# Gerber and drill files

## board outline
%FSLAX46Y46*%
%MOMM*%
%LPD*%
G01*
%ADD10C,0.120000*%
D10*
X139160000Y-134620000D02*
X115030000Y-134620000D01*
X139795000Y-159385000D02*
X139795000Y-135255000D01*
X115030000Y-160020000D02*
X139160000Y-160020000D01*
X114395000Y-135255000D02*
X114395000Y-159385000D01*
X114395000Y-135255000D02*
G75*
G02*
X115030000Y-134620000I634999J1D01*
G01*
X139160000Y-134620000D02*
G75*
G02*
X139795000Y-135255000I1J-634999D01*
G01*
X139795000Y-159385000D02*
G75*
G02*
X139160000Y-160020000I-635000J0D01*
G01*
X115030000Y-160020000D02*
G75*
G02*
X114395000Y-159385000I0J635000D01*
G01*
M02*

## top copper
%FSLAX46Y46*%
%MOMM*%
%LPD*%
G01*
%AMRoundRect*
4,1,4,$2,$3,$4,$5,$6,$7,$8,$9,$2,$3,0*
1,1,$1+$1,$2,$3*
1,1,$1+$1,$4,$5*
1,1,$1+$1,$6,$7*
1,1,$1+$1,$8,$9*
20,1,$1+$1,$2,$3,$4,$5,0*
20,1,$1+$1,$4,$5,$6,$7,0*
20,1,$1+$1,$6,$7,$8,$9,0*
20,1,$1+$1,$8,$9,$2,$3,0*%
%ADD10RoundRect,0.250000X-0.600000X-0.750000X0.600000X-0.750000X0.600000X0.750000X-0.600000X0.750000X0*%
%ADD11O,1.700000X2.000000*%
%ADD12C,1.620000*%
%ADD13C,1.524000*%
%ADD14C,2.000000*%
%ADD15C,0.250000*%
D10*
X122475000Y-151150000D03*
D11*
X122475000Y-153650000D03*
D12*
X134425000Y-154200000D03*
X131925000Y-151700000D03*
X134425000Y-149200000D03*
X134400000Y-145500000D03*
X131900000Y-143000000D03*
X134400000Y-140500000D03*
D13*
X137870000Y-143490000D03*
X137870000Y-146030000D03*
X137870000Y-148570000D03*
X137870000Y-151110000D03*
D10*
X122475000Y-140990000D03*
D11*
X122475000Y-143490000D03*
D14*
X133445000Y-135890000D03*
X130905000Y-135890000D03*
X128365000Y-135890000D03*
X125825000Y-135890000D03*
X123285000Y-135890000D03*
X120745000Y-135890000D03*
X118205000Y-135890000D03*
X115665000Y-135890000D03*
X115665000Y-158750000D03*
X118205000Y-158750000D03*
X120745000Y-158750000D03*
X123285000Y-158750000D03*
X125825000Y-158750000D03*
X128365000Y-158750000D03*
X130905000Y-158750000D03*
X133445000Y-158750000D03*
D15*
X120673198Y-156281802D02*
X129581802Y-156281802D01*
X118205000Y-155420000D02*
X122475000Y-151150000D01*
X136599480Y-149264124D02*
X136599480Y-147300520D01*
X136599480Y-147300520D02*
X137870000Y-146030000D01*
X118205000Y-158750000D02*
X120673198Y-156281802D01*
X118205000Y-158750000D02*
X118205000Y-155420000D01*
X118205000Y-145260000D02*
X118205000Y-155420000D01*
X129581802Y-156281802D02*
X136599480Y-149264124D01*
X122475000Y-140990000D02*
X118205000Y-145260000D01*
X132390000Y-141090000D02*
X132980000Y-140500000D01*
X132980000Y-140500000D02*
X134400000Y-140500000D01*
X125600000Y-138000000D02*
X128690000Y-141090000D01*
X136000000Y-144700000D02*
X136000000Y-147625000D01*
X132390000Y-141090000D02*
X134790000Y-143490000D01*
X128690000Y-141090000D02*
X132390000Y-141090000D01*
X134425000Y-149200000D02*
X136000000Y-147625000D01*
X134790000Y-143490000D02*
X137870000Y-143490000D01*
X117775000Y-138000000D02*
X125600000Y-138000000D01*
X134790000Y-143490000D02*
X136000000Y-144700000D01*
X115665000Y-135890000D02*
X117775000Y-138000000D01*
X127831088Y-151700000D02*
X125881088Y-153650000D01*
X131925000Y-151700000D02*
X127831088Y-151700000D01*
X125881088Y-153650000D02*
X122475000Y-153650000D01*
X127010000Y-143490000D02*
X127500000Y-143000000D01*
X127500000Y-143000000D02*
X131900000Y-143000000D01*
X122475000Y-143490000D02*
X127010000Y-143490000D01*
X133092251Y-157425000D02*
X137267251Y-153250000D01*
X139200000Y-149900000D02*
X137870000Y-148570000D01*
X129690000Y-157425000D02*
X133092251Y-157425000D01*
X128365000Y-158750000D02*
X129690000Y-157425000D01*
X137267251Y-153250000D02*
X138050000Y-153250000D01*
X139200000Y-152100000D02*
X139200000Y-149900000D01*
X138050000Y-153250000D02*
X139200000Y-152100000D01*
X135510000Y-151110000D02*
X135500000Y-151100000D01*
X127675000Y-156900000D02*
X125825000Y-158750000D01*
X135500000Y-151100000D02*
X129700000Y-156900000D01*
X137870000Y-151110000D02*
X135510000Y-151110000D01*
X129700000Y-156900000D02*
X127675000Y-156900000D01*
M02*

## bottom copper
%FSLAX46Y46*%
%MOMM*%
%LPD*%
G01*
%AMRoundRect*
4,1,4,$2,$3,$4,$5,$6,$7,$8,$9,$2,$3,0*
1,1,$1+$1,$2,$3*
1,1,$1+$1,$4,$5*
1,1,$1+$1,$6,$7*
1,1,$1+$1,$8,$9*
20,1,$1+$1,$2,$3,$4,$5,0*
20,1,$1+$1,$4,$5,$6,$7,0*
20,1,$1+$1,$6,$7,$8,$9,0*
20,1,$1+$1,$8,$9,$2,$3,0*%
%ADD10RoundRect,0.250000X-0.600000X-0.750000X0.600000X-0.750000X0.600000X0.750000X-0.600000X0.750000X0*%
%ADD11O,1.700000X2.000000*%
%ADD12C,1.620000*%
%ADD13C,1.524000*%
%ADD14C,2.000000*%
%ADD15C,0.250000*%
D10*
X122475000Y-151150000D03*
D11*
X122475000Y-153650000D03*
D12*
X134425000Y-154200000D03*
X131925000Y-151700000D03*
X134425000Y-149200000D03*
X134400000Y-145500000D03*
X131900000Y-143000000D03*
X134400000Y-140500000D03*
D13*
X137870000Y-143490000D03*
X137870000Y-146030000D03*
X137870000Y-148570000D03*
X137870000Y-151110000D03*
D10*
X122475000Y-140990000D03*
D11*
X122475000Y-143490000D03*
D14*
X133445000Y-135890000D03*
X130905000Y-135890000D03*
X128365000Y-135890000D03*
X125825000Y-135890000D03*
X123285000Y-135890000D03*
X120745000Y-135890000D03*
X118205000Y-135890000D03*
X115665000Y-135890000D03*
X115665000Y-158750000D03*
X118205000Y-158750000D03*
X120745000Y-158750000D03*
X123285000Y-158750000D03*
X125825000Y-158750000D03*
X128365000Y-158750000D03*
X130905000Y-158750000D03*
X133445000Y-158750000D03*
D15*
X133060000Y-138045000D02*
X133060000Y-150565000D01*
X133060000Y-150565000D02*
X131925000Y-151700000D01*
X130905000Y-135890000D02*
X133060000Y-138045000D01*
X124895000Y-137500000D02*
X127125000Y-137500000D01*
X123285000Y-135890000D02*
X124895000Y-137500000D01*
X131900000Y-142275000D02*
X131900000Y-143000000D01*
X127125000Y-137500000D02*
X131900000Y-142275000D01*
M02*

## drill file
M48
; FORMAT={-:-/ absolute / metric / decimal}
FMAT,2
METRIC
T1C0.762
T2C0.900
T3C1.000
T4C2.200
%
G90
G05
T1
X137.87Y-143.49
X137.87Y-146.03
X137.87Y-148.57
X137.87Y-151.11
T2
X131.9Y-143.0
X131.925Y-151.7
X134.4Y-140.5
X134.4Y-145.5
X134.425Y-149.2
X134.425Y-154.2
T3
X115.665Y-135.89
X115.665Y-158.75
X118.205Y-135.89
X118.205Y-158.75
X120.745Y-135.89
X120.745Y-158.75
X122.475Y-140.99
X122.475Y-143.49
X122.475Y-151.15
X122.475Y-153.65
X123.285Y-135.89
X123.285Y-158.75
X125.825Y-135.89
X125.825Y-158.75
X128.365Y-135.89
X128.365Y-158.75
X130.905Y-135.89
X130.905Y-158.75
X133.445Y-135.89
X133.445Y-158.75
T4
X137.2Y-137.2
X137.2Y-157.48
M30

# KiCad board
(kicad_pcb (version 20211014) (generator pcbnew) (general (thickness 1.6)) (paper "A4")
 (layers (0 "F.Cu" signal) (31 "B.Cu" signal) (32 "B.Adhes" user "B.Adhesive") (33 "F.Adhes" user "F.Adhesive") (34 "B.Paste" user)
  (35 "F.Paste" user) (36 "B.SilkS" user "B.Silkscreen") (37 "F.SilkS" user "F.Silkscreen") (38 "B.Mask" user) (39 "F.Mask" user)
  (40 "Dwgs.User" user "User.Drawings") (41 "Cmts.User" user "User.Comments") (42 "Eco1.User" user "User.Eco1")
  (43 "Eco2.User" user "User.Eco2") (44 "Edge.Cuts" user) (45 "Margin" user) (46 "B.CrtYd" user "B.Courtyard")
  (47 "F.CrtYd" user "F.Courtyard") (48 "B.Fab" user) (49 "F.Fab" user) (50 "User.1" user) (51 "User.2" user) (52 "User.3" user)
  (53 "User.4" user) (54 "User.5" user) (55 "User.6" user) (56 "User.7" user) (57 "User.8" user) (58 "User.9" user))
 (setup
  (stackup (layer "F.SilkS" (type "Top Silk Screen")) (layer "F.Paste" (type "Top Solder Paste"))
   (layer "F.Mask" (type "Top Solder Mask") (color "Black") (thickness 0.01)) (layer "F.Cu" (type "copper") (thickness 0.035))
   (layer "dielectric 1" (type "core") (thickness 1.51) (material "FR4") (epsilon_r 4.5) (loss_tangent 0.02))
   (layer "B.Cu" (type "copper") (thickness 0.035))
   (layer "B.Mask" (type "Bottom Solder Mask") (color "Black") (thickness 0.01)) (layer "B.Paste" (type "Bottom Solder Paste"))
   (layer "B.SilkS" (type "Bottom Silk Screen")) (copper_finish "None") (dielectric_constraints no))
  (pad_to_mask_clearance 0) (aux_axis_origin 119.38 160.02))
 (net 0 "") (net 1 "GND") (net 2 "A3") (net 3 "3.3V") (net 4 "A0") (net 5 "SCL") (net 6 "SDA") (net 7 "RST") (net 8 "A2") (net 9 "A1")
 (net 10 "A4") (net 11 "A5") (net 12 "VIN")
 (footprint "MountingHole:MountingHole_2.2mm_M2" (layer "F.Cu") (at 137.2 137.2)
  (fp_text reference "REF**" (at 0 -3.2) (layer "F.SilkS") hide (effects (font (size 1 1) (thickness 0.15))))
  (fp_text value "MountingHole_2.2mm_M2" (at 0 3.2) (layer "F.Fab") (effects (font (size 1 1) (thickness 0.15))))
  (pad "" np_thru_hole circle (at 0 0) (size 2.2 2.2) (drill 2.2) (layers *.Cu *.Mask)))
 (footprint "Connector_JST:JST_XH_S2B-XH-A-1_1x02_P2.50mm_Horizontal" (layer "F.Cu") (at 114.375 152.4 -90)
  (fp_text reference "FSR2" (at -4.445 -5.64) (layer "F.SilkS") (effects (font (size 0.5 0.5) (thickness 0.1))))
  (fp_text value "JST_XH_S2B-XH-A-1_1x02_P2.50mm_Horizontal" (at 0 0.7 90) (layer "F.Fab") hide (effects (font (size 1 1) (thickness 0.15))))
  (pad "1" thru_hole roundrect (at -1.25 -8.1) (size 1.7 2) (drill 1) (layers *.Cu *.Mask) (roundrect_rratio 0.1470588235) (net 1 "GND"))
  (pad "2" thru_hole oval (at 1.25 -8.1) (size 1.7 2) (drill 1) (layers *.Cu *.Mask) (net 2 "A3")))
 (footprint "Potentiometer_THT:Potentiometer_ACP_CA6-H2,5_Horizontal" (layer "F.Cu") (at 134.425 154.2 180)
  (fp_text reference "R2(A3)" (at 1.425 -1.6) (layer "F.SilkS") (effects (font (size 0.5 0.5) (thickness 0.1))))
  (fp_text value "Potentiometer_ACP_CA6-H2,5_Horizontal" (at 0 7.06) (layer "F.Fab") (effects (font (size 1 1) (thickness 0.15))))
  (pad "1" thru_hole circle (at 0 0 180) (size 1.62 1.62) (drill 0.9) (layers *.Cu *.Mask))
  (pad "2" thru_hole circle (at 2.5 2.5 180) (size 1.62 1.62) (drill 0.9) (layers *.Cu *.Mask) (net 2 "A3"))
  (pad "3" thru_hole circle (at 0 5 180) (size 1.62 1.62) (drill 0.9) (layers *.Cu *.Mask) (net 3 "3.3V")))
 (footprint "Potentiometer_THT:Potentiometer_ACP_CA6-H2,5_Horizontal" (layer "F.Cu") (at 134.4 145.5 180)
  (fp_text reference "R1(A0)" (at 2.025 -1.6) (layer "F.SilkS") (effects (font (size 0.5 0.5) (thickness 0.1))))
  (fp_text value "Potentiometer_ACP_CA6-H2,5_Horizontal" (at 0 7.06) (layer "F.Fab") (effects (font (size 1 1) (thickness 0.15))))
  (pad "1" thru_hole circle (at 0 0 180) (size 1.62 1.62) (drill 0.9) (layers *.Cu *.Mask))
  (pad "2" thru_hole circle (at 2.5 2.5 180) (size 1.62 1.62) (drill 0.9) (layers *.Cu *.Mask) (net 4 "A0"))
  (pad "3" thru_hole circle (at 0 5 180) (size 1.62 1.62) (drill 0.9) (layers *.Cu *.Mask) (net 3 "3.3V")))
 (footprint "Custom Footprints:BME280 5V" (layer "F.Cu") (at 136.6 147.3 -90)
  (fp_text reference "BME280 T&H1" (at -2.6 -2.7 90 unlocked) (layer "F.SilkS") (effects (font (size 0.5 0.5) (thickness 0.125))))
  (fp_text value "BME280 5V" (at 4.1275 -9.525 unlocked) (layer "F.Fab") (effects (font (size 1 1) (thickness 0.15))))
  (pad "1" thru_hole circle (at -3.81 -1.27 180) (size 1.524 1.524) (drill 0.762) (layers *.Cu *.Mask) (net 3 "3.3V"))
  (pad "2" thru_hole circle (at -1.27 -1.27 180) (size 1.524 1.524) (drill 0.762) (layers *.Cu *.Mask) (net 1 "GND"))
  (pad "3" thru_hole circle (at 1.27 -1.27 180) (size 1.524 1.524) (drill 0.762) (layers *.Cu *.Mask) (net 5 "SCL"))
  (pad "4" thru_hole circle (at 3.81 -1.27 180) (size 1.524 1.524) (drill 0.762) (layers *.Cu *.Mask) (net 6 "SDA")))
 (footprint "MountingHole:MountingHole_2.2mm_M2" (layer "F.Cu") (at 137.2 157.44)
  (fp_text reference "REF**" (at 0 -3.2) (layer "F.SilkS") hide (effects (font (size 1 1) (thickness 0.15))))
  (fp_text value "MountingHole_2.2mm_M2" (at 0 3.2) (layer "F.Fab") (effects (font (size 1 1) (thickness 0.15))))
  (pad "" np_thru_hole circle (at 0 0.04) (size 2.2 2.2) (drill 2.2) (layers F&B.Cu *.Mask)))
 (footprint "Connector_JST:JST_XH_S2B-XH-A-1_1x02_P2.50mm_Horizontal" (layer "F.Cu") (at 114.375 142.24 -90)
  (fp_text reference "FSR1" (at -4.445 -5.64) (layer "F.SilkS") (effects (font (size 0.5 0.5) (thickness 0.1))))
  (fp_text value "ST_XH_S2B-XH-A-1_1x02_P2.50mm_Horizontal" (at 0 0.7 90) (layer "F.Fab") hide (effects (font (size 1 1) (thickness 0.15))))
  (pad "1" thru_hole roundrect (at -1.25 -8.1) (size 1.7 2) (drill 1) (layers *.Cu *.Mask) (roundrect_rratio 0.1470588235) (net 1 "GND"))
  (pad "2" thru_hole oval (at 1.25 -8.1) (size 1.7 2) (drill 1) (layers *.Cu *.Mask) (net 4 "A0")))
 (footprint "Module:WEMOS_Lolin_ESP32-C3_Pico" (layer "F.Cu") (at 114.395 147.32 -90)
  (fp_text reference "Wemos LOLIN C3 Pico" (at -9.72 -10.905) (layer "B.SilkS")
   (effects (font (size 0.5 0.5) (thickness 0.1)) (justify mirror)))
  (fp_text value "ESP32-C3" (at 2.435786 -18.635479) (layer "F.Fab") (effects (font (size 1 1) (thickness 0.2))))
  (fp_line (start -12.7 -24.765) (end -12.7 -0.635) (layer "Edge.Cuts") (width 0.12))
  (fp_line (start 12.065 -25.4) (end -12.065 -25.4) (layer "Edge.Cuts") (width 0.12))
  (fp_line (start 12.7 -0.635) (end 12.7 -24.765) (layer "Edge.Cuts") (width 0.12))
  (fp_line (start -12.065 0) (end 12.065 0) (layer "Edge.Cuts") (width 0.12))
  (fp_arc (start -12.065 0) (mid -12.514013 -0.185987) (end -12.7 -0.635) (layer "Edge.Cuts") (width 0.12))
  (fp_arc (start -12.7 -24.765) (mid -12.514013 -25.214013) (end -12.065 -25.4) (layer "Edge.Cuts") (width 0.12))
  (fp_arc (start 12.065 -25.4) (mid 12.514013 -25.214013) (end 12.7 -24.765) (layer "Edge.Cuts") (width 0.12))
  (fp_arc (start 12.7 -0.635) (mid 12.514013 -0.185987) (end 12.065 0) (layer "Edge.Cuts") (width 0.12))
  (pad "1" thru_hole circle (at -11.43 -19.05 270) (size 2 2) (drill 1) (layers *.Cu *.Mask) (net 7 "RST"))
  (pad "2" thru_hole circle (at -11.43 -16.51 270) (size 2 2) (drill 1) (layers *.Cu *.Mask) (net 2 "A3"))
  (pad "3" thru_hole circle (at -11.43 -13.97 270) (size 2 2) (drill 1) (layers *.Cu *.Mask) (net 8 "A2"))
  (pad "4" thru_hole circle (at -11.43 -11.43 270) (size 2 2) (drill 1) (layers *.Cu *.Mask) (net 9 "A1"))
  (pad "5" thru_hole circle (at -11.43 -8.89 270) (size 2 2) (drill 1) (layers *.Cu *.Mask) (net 4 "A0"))
  (pad "6" thru_hole circle (at -11.43 -6.35 270) (size 2 2) (drill 1) (layers *.Cu *.Mask) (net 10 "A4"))
  (pad "7" thru_hole circle (at -11.43 -3.81 270) (size 2 2) (drill 1) (layers *.Cu *.Mask) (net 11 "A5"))
  (pad "8" thru_hole circle (at -11.43 -1.27 270) (size 2 2) (drill 1) (layers *.Cu *.Mask) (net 3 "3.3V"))
  (pad "9" thru_hole circle (at 11.43 -1.27 270) (size 2 2) (drill 1) (layers *.Cu *.Mask) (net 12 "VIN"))
  (pad "10" thru_hole circle (at 11.43 -3.81 270) (size 2 2) (drill 1) (layers *.Cu *.Mask) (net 1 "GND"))
  (pad "11" thru_hole circle (at 11.43 -6.35 270) (size 2 2) (drill 1) (layers *.Cu *.Mask))
  (pad "12" thru_hole circle (at 11.43 -8.89 270) (size 2 2) (drill 1) (layers *.Cu *.Mask))
  (pad "13" thru_hole circle (at 11.43 -11.43 270) (size 2 2) (drill 1) (layers *.Cu *.Mask) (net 6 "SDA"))
  (pad "14" thru_hole circle (at 11.43 -13.97 270) (size 2 2) (drill 1) (layers *.Cu *.Mask) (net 5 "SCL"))
  (pad "15" thru_hole circle (at 11.43 -16.51 270) (size 2 2) (drill 1) (layers *.Cu *.Mask))
  (pad "16" thru_hole circle (at 11.43 -19.05 270) (size 2 2) (drill 1) (layers *.Cu *.Mask)))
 (segment (start 120.673198 156.281802) (end 129.581802 156.281802) (width 0.25) (layer "F.Cu") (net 1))
 (segment (start 118.205 155.42) (end 122.475 151.15) (width 0.25) (layer "F.Cu") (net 1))
 (segment (start 136.59948 149.264124) (end 136.59948 147.30052) (width 0.25) (layer "F.Cu") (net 1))
 (segment (start 136.59948 147.30052) (end 137.87 146.03) (width 0.25) (layer "F.Cu") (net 1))
 (segment (start 118.205 158.75) (end 120.673198 156.281802) (width 0.25) (layer "F.Cu") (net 1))
 (segment (start 118.205 158.75) (end 118.205 155.42) (width 0.25) (layer "F.Cu") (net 1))
 (segment (start 118.205 145.26) (end 118.205 155.42) (width 0.25) (layer "F.Cu") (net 1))
 (segment (start 129.581802 156.281802) (end 136.59948 149.264124) (width 0.25) (layer "F.Cu") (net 1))
 (segment (start 122.475 140.99) (end 118.205 145.26) (width 0.25) (layer "F.Cu") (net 1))
 (segment (start 132.39 141.09) (end 132.98 140.5) (width 0.25) (layer "F.Cu") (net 3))
 (segment (start 132.98 140.5) (end 134.4 140.5) (width 0.25) (layer "F.Cu") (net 3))
 (segment (start 125.6 138) (end 128.69 141.09) (width 0.25) (layer "F.Cu") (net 3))
 (segment (start 136 144.7) (end 136 147.625) (width 0.25) (layer "F.Cu") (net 3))
 (segment (start 132.39 141.09) (end 134.79 143.49) (width 0.25) (layer "F.Cu") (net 3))
 (segment (start 128.69 141.09) (end 132.39 141.09) (width 0.25) (layer "F.Cu") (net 3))
 (segment (start 134.425 149.2) (end 136 147.625) (width 0.25) (layer "F.Cu") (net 3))
 (segment (start 134.79 143.49) (end 137.87 143.49) (width 0.25) (layer "F.Cu") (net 3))
 (segment (start 117.775 138) (end 125.6 138) (width 0.25) (layer "F.Cu") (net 3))
 (segment (start 134.79 143.49) (end 136 144.7) (width 0.25) (layer "F.Cu") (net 3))
 (segment (start 115.665 135.89) (end 117.775 138) (width 0.25) (layer "F.Cu") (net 3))
 (segment (start 127.831088 151.7) (end 125.881088 153.65) (width 0.25) (layer "F.Cu") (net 2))
 (segment (start 131.925 151.7) (end 127.831088 151.7) (width 0.25) (layer "F.Cu") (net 2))
 (segment (start 125.881088 153.65) (end 122.475 153.65) (width 0.25) (layer "F.Cu") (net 2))
 (segment (start 133.06 138.045) (end 133.06 150.565) (width 0.25) (layer "B.Cu") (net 2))
 (segment (start 133.06 150.565) (end 131.925 151.7) (width 0.25) (layer "B.Cu") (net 2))
 (segment (start 130.905 135.89) (end 133.06 138.045) (width 0.25) (layer "B.Cu") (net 2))
 (segment (start 127.01 143.49) (end 127.5 143) (width 0.25) (layer "F.Cu") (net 4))
 (segment (start 127.5 143) (end 131.9 143) (width 0.25) (layer "F.Cu") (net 4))
 (segment (start 122.475 143.49) (end 127.01 143.49) (width 0.25) (layer "F.Cu") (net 4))
 (segment (start 124.895 137.5) (end 127.125 137.5) (width 0.25) (layer "B.Cu") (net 4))
 (segment (start 123.285 135.89) (end 124.895 137.5) (width 0.25) (layer "B.Cu") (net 4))
 (segment (start 131.9 142.275) (end 131.9 143) (width 0.25) (layer "B.Cu") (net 4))
 (segment (start 127.125 137.5) (end 131.9 142.275) (width 0.25) (layer "B.Cu") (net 4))
 (segment (start 133.092251 157.425) (end 137.267251 153.25) (width 0.25) (layer "F.Cu") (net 5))
 (segment (start 139.2 149.9) (end 137.87 148.57) (width 0.25) (layer "F.Cu") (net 5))
 (segment (start 129.69 157.425) (end 133.092251 157.425) (width 0.25) (layer "F.Cu") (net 5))
 (segment (start 128.365 158.75) (end 129.69 157.425) (width 0.25) (layer "F.Cu") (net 5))
 (segment (start 137.267251 153.25) (end 138.05 153.25) (width 0.25) (layer "F.Cu") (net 5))
 (segment (start 139.2 152.1) (end 139.2 149.9) (width 0.25) (layer "F.Cu") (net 5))
 (segment (start 138.05 153.25) (end 139.2 152.1) (width 0.25) (layer "F.Cu") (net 5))
 (segment (start 135.51 151.11) (end 135.5 151.1) (width 0.25) (layer "F.Cu") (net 6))
 (segment (start 127.675 156.9) (end 125.825 158.75) (width 0.25) (layer "F.Cu") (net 6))
 (segment (start 135.5 151.1) (end 129.7 156.9) (width 0.25) (layer "F.Cu") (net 6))
 (segment (start 137.87 151.11) (end 135.51 151.11) (width 0.25) (layer "F.Cu") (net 6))
 (segment (start 129.7 156.9) (end 127.675 156.9) (width 0.25) (layer "F.Cu") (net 6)))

